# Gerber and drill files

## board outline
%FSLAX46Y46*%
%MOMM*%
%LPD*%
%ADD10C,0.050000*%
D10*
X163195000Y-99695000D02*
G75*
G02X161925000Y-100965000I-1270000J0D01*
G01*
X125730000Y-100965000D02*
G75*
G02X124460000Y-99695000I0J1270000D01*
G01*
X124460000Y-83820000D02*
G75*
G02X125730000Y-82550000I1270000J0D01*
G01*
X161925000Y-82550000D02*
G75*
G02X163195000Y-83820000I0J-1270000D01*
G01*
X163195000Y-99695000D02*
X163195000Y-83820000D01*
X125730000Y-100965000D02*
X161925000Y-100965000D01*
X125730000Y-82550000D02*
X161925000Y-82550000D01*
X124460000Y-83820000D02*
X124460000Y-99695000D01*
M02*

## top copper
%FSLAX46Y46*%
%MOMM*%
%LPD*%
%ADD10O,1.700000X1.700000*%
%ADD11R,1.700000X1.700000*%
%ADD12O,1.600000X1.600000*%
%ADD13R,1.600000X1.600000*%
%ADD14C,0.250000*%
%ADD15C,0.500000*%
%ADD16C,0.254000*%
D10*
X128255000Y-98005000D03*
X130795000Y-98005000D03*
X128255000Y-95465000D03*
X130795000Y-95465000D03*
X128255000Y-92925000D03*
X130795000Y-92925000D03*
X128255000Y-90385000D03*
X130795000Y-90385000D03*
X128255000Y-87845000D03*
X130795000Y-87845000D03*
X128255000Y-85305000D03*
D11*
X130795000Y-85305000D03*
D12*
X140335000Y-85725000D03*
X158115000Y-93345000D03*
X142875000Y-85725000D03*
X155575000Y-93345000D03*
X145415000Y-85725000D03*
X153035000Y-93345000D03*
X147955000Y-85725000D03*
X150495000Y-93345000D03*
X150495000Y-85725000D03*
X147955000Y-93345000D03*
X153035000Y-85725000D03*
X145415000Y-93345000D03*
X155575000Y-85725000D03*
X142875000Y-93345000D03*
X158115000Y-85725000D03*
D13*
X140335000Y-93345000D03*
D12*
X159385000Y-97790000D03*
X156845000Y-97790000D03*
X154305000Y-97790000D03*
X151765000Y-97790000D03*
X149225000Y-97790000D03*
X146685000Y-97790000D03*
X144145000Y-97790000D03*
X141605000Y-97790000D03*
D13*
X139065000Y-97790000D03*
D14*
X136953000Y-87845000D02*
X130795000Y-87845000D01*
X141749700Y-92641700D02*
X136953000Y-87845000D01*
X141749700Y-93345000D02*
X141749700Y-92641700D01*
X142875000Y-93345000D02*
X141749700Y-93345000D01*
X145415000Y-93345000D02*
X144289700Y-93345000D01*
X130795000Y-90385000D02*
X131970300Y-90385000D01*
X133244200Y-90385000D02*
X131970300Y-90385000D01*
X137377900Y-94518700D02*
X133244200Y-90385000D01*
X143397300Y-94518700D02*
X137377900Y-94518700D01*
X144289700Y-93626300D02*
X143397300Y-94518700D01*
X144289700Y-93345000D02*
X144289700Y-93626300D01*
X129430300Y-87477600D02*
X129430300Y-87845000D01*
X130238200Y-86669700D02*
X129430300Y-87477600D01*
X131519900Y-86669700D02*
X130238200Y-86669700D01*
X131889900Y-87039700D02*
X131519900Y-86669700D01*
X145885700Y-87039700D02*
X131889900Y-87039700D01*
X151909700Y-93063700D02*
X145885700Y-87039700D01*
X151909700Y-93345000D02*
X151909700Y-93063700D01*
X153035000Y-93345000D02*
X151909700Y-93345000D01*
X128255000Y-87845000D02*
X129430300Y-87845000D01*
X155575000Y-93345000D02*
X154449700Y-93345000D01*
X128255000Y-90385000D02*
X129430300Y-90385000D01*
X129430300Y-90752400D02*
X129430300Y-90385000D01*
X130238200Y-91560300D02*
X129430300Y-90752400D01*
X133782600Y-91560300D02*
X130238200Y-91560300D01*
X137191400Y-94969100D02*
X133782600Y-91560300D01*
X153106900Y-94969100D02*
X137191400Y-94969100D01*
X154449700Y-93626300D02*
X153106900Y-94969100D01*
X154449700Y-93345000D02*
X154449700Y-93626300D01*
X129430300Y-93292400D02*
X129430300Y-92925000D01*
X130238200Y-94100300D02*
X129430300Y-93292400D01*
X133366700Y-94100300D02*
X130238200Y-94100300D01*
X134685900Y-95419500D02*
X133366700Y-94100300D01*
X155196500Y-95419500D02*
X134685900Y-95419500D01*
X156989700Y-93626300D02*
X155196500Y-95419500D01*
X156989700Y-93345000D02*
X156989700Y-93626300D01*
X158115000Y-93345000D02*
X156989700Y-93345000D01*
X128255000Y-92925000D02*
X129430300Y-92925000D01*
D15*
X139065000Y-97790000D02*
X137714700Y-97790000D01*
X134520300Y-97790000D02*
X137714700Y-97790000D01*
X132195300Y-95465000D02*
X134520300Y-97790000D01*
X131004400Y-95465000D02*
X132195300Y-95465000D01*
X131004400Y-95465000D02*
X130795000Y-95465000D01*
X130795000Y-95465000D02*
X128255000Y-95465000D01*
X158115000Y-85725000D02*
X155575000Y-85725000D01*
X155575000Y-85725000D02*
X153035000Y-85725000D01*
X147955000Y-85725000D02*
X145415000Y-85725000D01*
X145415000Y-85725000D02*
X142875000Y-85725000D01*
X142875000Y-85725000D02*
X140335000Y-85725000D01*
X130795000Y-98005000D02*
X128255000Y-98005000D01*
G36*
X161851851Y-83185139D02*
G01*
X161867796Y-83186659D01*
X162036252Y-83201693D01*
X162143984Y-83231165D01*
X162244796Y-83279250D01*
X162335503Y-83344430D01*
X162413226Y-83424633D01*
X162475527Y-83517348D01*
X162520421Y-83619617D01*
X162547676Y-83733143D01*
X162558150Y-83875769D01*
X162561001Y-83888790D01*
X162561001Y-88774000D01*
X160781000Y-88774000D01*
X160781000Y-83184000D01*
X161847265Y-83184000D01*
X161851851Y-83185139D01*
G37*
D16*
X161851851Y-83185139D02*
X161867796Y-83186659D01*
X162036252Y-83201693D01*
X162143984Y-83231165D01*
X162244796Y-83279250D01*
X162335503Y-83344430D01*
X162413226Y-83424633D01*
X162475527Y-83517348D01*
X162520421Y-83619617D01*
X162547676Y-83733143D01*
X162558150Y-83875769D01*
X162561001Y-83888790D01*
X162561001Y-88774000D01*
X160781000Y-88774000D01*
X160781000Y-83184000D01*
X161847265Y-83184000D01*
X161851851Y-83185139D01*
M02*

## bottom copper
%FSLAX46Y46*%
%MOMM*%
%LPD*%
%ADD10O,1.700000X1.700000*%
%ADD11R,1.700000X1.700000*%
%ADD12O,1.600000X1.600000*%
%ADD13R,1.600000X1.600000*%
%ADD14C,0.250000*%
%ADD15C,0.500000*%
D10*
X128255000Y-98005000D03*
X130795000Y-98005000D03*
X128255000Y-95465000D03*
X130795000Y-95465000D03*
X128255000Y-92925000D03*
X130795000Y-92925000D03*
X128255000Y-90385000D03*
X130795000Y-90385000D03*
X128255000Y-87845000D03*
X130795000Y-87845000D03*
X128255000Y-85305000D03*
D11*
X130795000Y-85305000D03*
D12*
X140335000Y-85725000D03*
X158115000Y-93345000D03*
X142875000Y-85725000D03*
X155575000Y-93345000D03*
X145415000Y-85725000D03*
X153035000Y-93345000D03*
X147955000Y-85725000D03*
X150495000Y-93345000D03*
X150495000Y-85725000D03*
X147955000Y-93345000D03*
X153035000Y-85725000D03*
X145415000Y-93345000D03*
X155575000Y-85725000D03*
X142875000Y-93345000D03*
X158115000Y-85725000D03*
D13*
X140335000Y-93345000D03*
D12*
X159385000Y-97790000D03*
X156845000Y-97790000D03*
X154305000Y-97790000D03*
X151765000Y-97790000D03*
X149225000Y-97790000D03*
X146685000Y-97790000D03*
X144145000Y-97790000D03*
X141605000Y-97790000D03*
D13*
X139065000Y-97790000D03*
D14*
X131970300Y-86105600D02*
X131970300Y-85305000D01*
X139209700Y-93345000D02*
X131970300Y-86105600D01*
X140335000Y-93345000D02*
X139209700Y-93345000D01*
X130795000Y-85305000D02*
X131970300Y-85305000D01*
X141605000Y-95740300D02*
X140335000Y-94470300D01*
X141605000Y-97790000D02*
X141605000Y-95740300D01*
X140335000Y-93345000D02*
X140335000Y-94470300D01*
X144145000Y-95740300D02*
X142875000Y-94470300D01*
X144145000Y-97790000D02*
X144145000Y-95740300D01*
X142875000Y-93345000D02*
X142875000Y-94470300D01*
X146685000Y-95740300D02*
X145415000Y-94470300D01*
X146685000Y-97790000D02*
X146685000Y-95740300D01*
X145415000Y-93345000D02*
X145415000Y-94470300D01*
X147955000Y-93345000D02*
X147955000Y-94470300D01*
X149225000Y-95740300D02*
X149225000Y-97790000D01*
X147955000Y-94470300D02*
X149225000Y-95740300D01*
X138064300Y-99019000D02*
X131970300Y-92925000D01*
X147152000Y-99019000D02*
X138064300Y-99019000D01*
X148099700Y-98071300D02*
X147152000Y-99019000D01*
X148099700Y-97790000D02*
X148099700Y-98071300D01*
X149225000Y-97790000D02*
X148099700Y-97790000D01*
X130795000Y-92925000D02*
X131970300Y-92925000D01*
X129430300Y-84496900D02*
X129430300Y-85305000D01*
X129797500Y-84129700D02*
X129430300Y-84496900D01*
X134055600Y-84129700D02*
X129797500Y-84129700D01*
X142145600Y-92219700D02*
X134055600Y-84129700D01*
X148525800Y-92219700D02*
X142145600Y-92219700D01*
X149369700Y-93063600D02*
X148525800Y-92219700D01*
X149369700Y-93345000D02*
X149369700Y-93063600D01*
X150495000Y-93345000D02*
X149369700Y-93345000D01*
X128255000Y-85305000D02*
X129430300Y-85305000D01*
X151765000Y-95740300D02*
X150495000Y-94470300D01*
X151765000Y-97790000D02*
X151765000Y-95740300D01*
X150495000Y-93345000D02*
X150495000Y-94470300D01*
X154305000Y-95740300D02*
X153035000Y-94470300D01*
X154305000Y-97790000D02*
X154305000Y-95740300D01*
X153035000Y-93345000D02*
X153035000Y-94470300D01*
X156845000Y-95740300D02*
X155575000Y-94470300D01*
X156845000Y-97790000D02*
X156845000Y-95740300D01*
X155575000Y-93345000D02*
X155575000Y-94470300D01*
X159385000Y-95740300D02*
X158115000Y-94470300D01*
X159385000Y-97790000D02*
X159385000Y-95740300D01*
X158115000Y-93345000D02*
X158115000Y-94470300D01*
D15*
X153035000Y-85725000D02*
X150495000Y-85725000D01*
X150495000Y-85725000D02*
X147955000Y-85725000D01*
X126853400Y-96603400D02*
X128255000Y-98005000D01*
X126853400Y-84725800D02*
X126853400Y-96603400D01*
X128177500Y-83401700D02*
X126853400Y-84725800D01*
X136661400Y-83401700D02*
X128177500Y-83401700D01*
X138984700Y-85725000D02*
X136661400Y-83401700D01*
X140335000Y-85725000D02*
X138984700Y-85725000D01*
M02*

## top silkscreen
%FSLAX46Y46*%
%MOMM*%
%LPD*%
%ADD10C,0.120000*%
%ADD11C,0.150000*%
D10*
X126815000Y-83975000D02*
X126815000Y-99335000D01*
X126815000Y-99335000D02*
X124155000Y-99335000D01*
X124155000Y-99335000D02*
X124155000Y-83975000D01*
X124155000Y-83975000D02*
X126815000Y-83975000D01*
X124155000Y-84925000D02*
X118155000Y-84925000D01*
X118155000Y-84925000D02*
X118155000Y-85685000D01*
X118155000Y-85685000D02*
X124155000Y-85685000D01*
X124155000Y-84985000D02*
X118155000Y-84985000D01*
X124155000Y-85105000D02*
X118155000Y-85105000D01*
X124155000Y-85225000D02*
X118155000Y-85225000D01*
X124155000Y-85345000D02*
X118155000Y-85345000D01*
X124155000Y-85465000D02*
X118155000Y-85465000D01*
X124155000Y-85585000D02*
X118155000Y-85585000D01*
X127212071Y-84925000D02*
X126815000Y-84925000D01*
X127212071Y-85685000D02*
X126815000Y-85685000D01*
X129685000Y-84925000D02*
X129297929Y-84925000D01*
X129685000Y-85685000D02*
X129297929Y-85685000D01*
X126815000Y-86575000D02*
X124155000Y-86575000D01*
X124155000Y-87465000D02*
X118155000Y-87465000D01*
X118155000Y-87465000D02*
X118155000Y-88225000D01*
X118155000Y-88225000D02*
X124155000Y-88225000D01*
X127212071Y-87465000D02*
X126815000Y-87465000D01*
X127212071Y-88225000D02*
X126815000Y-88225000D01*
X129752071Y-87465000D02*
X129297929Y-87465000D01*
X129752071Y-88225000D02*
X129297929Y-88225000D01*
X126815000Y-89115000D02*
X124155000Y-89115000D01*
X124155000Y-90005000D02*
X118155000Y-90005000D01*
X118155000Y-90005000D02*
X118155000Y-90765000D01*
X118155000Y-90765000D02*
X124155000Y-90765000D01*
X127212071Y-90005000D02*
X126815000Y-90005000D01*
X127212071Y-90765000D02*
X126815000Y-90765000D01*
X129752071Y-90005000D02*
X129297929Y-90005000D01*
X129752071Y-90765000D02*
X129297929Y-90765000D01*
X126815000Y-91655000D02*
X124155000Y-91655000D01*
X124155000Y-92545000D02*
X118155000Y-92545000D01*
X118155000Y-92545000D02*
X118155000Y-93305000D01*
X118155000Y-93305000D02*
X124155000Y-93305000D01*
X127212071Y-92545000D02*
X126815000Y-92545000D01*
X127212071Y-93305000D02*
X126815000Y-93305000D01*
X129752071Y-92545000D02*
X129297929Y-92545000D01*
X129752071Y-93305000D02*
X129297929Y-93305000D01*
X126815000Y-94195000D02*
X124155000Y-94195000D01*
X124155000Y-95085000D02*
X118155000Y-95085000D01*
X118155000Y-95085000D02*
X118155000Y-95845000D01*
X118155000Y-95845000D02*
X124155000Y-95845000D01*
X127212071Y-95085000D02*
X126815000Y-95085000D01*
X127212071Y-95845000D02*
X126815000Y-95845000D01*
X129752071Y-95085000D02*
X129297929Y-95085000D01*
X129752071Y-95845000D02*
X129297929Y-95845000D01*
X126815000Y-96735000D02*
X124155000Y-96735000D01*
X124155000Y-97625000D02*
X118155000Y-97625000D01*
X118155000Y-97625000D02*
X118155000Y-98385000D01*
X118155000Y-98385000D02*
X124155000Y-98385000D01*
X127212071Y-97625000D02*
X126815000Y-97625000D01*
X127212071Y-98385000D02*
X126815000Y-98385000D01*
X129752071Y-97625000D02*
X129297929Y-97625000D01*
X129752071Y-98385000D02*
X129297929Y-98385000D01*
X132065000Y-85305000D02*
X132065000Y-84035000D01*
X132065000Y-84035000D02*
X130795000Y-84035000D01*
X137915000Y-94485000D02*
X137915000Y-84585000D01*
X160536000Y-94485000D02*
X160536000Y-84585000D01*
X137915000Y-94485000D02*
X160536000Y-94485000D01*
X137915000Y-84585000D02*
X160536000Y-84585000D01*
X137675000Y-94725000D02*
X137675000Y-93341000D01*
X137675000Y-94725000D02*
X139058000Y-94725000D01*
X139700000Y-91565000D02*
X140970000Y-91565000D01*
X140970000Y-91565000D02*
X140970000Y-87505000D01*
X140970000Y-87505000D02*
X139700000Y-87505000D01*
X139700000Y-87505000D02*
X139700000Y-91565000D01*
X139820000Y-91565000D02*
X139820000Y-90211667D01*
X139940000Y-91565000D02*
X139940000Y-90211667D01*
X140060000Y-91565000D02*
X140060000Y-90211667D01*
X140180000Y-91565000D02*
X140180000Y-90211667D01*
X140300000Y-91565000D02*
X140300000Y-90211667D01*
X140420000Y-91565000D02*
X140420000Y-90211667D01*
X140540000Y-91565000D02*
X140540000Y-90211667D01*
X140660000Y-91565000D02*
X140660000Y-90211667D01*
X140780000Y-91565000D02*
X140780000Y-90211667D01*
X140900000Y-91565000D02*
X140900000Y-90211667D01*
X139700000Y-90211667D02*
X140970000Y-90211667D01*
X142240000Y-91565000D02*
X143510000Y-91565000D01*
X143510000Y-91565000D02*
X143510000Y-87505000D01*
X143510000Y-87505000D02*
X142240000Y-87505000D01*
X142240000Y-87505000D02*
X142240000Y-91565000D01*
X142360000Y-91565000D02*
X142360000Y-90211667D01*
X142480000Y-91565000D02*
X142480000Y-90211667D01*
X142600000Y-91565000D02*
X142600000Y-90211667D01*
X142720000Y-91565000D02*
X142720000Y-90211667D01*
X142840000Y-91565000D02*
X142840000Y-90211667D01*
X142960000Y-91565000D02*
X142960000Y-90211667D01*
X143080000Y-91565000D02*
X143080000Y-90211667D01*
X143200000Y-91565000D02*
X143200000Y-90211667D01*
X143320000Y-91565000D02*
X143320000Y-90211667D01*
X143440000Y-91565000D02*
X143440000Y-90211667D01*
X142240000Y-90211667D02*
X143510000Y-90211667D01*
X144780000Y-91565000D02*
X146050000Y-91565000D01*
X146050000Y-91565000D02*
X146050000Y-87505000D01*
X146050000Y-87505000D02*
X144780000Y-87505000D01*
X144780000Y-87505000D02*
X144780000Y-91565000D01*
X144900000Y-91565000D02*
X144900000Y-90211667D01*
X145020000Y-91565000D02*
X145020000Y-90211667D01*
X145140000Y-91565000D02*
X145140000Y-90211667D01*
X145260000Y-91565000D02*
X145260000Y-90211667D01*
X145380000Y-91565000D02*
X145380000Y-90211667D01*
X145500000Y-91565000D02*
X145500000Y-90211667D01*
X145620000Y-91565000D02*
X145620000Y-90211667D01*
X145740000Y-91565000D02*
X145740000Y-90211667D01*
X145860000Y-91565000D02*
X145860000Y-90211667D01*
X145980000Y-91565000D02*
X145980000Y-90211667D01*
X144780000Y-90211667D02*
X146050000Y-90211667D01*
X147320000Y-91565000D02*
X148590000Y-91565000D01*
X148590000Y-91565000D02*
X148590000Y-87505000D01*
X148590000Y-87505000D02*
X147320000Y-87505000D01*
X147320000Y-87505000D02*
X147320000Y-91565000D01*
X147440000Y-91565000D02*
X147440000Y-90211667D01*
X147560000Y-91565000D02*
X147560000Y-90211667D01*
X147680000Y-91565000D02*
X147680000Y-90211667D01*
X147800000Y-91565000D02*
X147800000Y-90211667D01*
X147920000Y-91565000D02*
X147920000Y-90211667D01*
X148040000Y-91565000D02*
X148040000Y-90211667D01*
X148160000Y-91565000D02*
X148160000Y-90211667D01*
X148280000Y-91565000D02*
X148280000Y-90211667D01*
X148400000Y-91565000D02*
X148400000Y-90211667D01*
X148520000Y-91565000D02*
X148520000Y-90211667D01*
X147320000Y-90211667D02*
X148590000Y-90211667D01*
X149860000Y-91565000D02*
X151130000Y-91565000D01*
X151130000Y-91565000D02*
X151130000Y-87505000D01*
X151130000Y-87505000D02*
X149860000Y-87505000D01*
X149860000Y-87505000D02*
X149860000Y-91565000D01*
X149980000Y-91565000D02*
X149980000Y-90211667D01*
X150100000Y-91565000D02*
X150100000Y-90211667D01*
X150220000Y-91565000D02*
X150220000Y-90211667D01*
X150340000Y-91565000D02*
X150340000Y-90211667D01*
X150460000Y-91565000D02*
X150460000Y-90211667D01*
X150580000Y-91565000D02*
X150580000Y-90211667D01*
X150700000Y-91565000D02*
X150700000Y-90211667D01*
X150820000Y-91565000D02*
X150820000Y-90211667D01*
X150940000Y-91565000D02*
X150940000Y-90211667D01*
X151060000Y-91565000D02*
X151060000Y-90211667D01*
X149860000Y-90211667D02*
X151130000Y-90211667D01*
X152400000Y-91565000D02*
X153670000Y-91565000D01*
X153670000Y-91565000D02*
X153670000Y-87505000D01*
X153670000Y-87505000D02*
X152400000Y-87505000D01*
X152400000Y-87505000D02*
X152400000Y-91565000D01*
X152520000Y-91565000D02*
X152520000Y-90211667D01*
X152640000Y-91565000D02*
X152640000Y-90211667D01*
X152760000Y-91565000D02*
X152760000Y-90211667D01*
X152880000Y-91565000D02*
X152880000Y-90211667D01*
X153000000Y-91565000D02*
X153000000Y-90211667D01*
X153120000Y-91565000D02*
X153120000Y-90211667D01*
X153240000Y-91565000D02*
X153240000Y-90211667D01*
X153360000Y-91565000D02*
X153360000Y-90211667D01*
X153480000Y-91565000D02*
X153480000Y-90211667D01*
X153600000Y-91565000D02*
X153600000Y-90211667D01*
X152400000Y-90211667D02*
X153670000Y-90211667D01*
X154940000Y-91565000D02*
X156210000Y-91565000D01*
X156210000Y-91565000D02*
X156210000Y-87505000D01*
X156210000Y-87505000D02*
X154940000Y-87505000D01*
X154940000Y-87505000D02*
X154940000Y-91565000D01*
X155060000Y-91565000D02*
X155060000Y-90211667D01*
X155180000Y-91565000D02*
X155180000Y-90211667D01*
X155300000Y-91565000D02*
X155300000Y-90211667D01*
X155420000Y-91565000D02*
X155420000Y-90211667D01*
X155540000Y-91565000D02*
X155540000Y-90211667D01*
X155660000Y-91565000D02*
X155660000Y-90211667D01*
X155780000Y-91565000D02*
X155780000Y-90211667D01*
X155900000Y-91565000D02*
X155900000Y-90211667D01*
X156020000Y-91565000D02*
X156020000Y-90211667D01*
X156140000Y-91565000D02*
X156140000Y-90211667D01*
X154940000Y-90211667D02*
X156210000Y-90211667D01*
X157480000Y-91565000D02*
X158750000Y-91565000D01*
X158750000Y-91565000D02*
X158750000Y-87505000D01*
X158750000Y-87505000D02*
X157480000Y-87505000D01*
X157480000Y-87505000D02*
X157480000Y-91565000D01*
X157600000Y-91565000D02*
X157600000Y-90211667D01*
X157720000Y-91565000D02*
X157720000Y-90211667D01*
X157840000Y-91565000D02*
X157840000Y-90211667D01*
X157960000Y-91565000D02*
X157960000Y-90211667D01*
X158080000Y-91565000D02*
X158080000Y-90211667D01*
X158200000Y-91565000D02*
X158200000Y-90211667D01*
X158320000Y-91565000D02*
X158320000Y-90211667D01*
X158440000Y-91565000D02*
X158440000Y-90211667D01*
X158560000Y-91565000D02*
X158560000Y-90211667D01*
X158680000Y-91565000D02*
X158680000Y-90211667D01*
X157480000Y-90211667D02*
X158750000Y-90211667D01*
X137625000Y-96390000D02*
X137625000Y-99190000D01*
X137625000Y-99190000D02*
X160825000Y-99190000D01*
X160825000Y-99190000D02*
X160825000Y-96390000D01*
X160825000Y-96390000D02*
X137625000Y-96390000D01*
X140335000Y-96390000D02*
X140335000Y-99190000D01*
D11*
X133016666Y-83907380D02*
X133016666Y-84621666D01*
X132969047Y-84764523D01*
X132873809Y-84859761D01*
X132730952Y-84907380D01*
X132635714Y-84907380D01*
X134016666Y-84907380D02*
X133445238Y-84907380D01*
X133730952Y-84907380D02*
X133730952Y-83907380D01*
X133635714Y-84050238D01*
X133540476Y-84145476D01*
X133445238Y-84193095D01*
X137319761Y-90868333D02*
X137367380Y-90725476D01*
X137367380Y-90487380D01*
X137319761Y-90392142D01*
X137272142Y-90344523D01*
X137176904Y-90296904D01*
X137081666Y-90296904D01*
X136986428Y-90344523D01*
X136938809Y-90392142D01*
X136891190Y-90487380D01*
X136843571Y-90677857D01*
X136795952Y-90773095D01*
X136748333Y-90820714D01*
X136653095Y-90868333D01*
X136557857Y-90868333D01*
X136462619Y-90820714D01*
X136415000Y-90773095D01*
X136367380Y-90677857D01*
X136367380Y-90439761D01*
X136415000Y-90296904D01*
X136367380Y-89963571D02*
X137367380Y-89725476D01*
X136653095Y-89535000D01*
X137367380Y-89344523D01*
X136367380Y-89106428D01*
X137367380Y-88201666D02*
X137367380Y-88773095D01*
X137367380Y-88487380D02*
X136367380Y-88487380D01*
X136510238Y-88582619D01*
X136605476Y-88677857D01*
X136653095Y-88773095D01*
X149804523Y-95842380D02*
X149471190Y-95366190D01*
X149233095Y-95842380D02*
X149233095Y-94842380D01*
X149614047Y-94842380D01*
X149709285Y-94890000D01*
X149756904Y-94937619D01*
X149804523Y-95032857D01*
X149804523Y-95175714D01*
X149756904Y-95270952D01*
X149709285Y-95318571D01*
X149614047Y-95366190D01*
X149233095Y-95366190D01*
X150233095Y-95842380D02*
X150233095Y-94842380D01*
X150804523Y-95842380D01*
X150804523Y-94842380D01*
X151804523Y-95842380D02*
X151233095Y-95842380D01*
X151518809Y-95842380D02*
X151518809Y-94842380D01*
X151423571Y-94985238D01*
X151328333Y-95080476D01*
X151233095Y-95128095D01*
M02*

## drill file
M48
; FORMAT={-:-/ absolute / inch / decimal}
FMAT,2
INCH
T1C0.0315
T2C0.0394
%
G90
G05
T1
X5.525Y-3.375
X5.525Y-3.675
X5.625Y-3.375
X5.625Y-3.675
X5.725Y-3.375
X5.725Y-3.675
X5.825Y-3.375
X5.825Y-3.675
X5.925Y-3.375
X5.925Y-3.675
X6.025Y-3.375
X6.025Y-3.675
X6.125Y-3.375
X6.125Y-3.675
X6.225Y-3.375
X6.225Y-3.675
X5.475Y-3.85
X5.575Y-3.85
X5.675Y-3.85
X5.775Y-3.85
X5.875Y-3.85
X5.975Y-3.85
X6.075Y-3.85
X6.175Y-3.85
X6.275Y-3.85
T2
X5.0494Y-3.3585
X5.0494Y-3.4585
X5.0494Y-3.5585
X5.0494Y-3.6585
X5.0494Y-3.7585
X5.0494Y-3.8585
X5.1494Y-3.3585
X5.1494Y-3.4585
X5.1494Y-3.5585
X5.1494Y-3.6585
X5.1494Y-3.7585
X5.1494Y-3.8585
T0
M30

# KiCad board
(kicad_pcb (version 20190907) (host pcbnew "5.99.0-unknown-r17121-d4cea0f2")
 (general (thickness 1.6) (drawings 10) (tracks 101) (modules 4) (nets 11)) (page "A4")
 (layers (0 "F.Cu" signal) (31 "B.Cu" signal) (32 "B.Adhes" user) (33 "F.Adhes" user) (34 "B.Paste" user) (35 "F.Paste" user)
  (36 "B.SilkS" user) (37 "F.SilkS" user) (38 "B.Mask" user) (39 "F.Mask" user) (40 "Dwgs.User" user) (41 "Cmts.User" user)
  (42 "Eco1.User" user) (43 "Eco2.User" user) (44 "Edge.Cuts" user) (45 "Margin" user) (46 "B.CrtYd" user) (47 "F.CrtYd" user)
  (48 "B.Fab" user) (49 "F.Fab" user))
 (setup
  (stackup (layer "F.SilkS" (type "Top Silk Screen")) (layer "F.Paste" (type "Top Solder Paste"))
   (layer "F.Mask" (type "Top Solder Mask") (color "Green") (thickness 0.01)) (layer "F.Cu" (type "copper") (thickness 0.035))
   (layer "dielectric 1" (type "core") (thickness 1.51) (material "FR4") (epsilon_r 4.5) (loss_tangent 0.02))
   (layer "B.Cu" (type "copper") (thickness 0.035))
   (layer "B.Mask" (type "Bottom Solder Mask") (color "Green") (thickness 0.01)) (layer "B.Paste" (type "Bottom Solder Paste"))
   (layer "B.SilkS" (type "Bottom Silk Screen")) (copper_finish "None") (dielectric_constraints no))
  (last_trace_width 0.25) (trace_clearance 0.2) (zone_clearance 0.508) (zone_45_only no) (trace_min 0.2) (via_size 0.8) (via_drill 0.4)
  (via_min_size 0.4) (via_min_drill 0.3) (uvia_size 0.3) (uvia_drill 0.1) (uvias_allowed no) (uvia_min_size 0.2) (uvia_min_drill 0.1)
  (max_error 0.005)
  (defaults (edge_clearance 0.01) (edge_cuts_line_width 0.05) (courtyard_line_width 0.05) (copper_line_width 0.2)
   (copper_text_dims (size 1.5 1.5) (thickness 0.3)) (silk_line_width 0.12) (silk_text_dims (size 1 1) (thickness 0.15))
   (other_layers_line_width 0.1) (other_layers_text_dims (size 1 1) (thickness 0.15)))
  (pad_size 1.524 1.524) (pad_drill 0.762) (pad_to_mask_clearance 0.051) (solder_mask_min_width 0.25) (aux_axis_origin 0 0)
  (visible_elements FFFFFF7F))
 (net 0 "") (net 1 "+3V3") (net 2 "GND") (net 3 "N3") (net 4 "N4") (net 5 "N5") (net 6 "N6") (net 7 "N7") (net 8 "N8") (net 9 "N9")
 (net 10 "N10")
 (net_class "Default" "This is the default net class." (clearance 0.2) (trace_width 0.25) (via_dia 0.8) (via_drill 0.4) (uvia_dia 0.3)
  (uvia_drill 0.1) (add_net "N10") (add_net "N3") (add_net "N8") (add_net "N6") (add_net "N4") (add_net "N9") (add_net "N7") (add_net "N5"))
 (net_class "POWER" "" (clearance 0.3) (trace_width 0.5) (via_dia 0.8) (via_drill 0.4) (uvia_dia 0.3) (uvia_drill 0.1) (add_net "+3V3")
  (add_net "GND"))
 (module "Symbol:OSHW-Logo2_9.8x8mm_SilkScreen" (layer "B.Cu") (at 135.255 91.694 -90)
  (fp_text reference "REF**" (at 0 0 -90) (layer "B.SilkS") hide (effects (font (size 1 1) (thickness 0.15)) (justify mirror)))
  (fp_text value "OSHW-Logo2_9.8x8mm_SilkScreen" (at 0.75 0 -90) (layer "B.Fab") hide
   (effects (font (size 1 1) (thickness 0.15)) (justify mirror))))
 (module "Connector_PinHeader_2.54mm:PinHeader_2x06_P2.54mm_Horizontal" (layer "F.Cu") (at 125.095 90.805)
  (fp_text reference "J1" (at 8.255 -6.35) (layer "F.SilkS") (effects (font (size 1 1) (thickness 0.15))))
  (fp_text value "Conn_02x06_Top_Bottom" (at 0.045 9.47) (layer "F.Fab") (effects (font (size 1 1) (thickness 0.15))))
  (fp_line (start 1.72 -6.83) (end 1.72 8.53) (layer "F.SilkS") (width 0.12))
  (fp_line (start 1.72 8.53) (end -0.94 8.53) (layer "F.SilkS") (width 0.12))
  (fp_line (start -0.94 8.53) (end -0.94 -6.83) (layer "F.SilkS") (width 0.12))
  (fp_line (start -0.94 -6.83) (end 1.72 -6.83) (layer "F.SilkS") (width 0.12))
  (fp_line (start -0.94 -5.88) (end -6.94 -5.88) (layer "F.SilkS") (width 0.12))
  (fp_line (start -6.94 -5.88) (end -6.94 -5.12) (layer "F.SilkS") (width 0.12))
  (fp_line (start -6.94 -5.12) (end -0.94 -5.12) (layer "F.SilkS") (width 0.12))
  (fp_line (start -0.94 -5.82) (end -6.94 -5.82) (layer "F.SilkS") (width 0.12))
  (fp_line (start -0.94 -5.7) (end -6.94 -5.7) (layer "F.SilkS") (width 0.12))
  (fp_line (start -0.94 -5.58) (end -6.94 -5.58) (layer "F.SilkS") (width 0.12))
  (fp_line (start -0.94 -5.46) (end -6.94 -5.46) (layer "F.SilkS") (width 0.12))
  (fp_line (start -0.94 -5.34) (end -6.94 -5.34) (layer "F.SilkS") (width 0.12))
  (fp_line (start -0.94 -5.22) (end -6.94 -5.22) (layer "F.SilkS") (width 0.12))
  (fp_line (start 2.117071 -5.88) (end 1.72 -5.88) (layer "F.SilkS") (width 0.12))
  (fp_line (start 2.117071 -5.12) (end 1.72 -5.12) (layer "F.SilkS") (width 0.12))
  (fp_line (start 4.59 -5.88) (end 4.202929 -5.88) (layer "F.SilkS") (width 0.12))
  (fp_line (start 4.59 -5.12) (end 4.202929 -5.12) (layer "F.SilkS") (width 0.12))
  (fp_line (start 1.72 -4.23) (end -0.94 -4.23) (layer "F.SilkS") (width 0.12))
  (fp_line (start -0.94 -3.34) (end -6.94 -3.34) (layer "F.SilkS") (width 0.12))
  (fp_line (start -6.94 -3.34) (end -6.94 -2.58) (layer "F.SilkS") (width 0.12))
  (fp_line (start -6.94 -2.58) (end -0.94 -2.58) (layer "F.SilkS") (width 0.12))
  (fp_line (start 2.117071 -3.34) (end 1.72 -3.34) (layer "F.SilkS") (width 0.12))
  (fp_line (start 2.117071 -2.58) (end 1.72 -2.58) (layer "F.SilkS") (width 0.12))
  (fp_line (start 4.657071 -3.34) (end 4.202929 -3.34) (layer "F.SilkS") (width 0.12))
  (fp_line (start 4.657071 -2.58) (end 4.202929 -2.58) (layer "F.SilkS") (width 0.12))
  (fp_line (start 1.72 -1.69) (end -0.94 -1.69) (layer "F.SilkS") (width 0.12))
  (fp_line (start -0.94 -0.8) (end -6.94 -0.8) (layer "F.SilkS") (width 0.12))
  (fp_line (start -6.94 -0.8) (end -6.94 -0.04) (layer "F.SilkS") (width 0.12))
  (fp_line (start -6.94 -0.04) (end -0.94 -0.04) (layer "F.SilkS") (width 0.12))
  (fp_line (start 2.117071 -0.8) (end 1.72 -0.8) (layer "F.SilkS") (width 0.12))
  (fp_line (start 2.117071 -0.04) (end 1.72 -0.04) (layer "F.SilkS") (width 0.12))
  (fp_line (start 4.657071 -0.8) (end 4.202929 -0.8) (layer "F.SilkS") (width 0.12))
  (fp_line (start 4.657071 -0.04) (end 4.202929 -0.04) (layer "F.SilkS") (width 0.12))
  (fp_line (start 1.72 0.85) (end -0.94 0.85) (layer "F.SilkS") (width 0.12))
  (fp_line (start -0.94 1.74) (end -6.94 1.74) (layer "F.SilkS") (width 0.12))
  (fp_line (start -6.94 1.74) (end -6.94 2.5) (layer "F.SilkS") (width 0.12))
  (fp_line (start -6.94 2.5) (end -0.94 2.5) (layer "F.SilkS") (width 0.12))
  (fp_line (start 2.117071 1.74) (end 1.72 1.74) (layer "F.SilkS") (width 0.12))
  (fp_line (start 2.117071 2.5) (end 1.72 2.5) (layer "F.SilkS") (width 0.12))
  (fp_line (start 4.657071 1.74) (end 4.202929 1.74) (layer "F.SilkS") (width 0.12))
  (fp_line (start 4.657071 2.5) (end 4.202929 2.5) (layer "F.SilkS") (width 0.12))
  (fp_line (start 1.72 3.39) (end -0.94 3.39) (layer "F.SilkS") (width 0.12))
  (fp_line (start -0.94 4.28) (end -6.94 4.28) (layer "F.SilkS") (width 0.12))
  (fp_line (start -6.94 4.28) (end -6.94 5.04) (layer "F.SilkS") (width 0.12))
  (fp_line (start -6.94 5.04) (end -0.94 5.04) (layer "F.SilkS") (width 0.12))
  (fp_line (start 2.117071 4.28) (end 1.72 4.28) (layer "F.SilkS") (width 0.12))
  (fp_line (start 2.117071 5.04) (end 1.72 5.04) (layer "F.SilkS") (width 0.12))
  (fp_line (start 4.657071 4.28) (end 4.202929 4.28) (layer "F.SilkS") (width 0.12))
  (fp_line (start 4.657071 5.04) (end 4.202929 5.04) (layer "F.SilkS") (width 0.12))
  (fp_line (start 1.72 5.93) (end -0.94 5.93) (layer "F.SilkS") (width 0.12))
  (fp_line (start -0.94 6.82) (end -6.94 6.82) (layer "F.SilkS") (width 0.12))
  (fp_line (start -6.94 6.82) (end -6.94 7.58) (layer "F.SilkS") (width 0.12))
  (fp_line (start -6.94 7.58) (end -0.94 7.58) (layer "F.SilkS") (width 0.12))
  (fp_line (start 2.117071 6.82) (end 1.72 6.82) (layer "F.SilkS") (width 0.12))
  (fp_line (start 2.117071 7.58) (end 1.72 7.58) (layer "F.SilkS") (width 0.12))
  (fp_line (start 4.657071 6.82) (end 4.202929 6.82) (layer "F.SilkS") (width 0.12))
  (fp_line (start 4.657071 7.58) (end 4.202929 7.58) (layer "F.SilkS") (width 0.12))
  (fp_line (start 6.97 -5.5) (end 6.97 -6.77) (layer "F.SilkS") (width 0.12))
  (fp_line (start 6.97 -6.77) (end 5.7 -6.77) (layer "F.SilkS") (width 0.12))
  (pad "12" thru_hole oval (at 3.16 7.2) (size 1.7 1.7) (drill 1) (layers *.Cu *.Mask) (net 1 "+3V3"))
  (pad "6" thru_hole oval (at 5.7 7.2) (size 1.7 1.7) (drill 1) (layers *.Cu *.Mask) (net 1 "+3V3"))
  (pad "11" thru_hole oval (at 3.16 4.66) (size 1.7 1.7) (drill 1) (layers *.Cu *.Mask) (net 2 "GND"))
  (pad "5" thru_hole oval (at 5.7 4.66) (size 1.7 1.7) (drill 1) (layers *.Cu *.Mask) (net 2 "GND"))
  (pad "10" thru_hole oval (at 3.16 2.12) (size 1.7 1.7) (drill 1) (layers *.Cu *.Mask) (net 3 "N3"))
  (pad "4" thru_hole oval (at 5.7 2.12) (size 1.7 1.7) (drill 1) (layers *.Cu *.Mask) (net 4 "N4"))
  (pad "9" thru_hole oval (at 3.16 -0.42) (size 1.7 1.7) (drill 1) (layers *.Cu *.Mask) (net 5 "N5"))
  (pad "3" thru_hole oval (at 5.7 -0.42) (size 1.7 1.7) (drill 1) (layers *.Cu *.Mask) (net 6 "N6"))
  (pad "8" thru_hole oval (at 3.16 -2.96) (size 1.7 1.7) (drill 1) (layers *.Cu *.Mask) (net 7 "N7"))
  (pad "2" thru_hole oval (at 5.7 -2.96) (size 1.7 1.7) (drill 1) (layers *.Cu *.Mask) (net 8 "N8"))
  (pad "7" thru_hole oval (at 3.16 -5.5) (size 1.7 1.7) (drill 1) (layers *.Cu *.Mask) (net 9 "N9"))
  (pad "1" thru_hole rect (at 5.7 -5.5) (size 1.7 1.7) (drill 1) (layers *.Cu *.Mask) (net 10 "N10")))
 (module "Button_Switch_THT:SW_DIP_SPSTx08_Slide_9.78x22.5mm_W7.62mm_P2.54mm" (layer "F.Cu") (at 140.335 93.345 90)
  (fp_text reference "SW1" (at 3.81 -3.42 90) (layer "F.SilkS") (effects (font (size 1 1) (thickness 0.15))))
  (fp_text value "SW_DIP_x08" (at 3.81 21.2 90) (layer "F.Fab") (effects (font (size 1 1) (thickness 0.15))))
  (fp_line (start -1.14 -2.42) (end 8.76 -2.42) (layer "F.SilkS") (width 0.12))
  (fp_line (start -1.14 20.201) (end 8.76 20.201) (layer "F.SilkS") (width 0.12))
  (fp_line (start -1.14 -2.42) (end -1.14 20.201) (layer "F.SilkS") (width 0.12))
  (fp_line (start 8.76 -2.42) (end 8.76 20.201) (layer "F.SilkS") (width 0.12))
  (fp_line (start -1.38 -2.66) (end 0.004 -2.66) (layer "F.SilkS") (width 0.12))
  (fp_line (start -1.38 -2.66) (end -1.38 -1.277) (layer "F.SilkS") (width 0.12))
  (fp_line (start 1.78 -0.635) (end 1.78 0.635) (layer "F.SilkS") (width 0.12))
  (fp_line (start 1.78 0.635) (end 5.84 0.635) (layer "F.SilkS") (width 0.12))
  (fp_line (start 5.84 0.635) (end 5.84 -0.635) (layer "F.SilkS") (width 0.12))
  (fp_line (start 5.84 -0.635) (end 1.78 -0.635) (layer "F.SilkS") (width 0.12))
  (fp_line (start 1.78 -0.515) (end 3.133333 -0.515) (layer "F.SilkS") (width 0.12))
  (fp_line (start 1.78 -0.395) (end 3.133333 -0.395) (layer "F.SilkS") (width 0.12))
  (fp_line (start 1.78 -0.275) (end 3.133333 -0.275) (layer "F.SilkS") (width 0.12))
  (fp_line (start 1.78 -0.155) (end 3.133333 -0.155) (layer "F.SilkS") (width 0.12))
  (fp_line (start 1.78 -0.035) (end 3.133333 -0.035) (layer "F.SilkS") (width 0.12))
  (fp_line (start 1.78 0.085) (end 3.133333 0.085) (layer "F.SilkS") (width 0.12))
  (fp_line (start 1.78 0.205) (end 3.133333 0.205) (layer "F.SilkS") (width 0.12))
  (fp_line (start 1.78 0.325) (end 3.133333 0.325) (layer "F.SilkS") (width 0.12))
  (fp_line (start 1.78 0.445) (end 3.133333 0.445) (layer "F.SilkS") (width 0.12))
  (fp_line (start 1.78 0.565) (end 3.133333 0.565) (layer "F.SilkS") (width 0.12))
  (fp_line (start 3.133333 -0.635) (end 3.133333 0.635) (layer "F.SilkS") (width 0.12))
  (fp_line (start 1.78 1.905) (end 1.78 3.175) (layer "F.SilkS") (width 0.12))
  (fp_line (start 1.78 3.175) (end 5.84 3.175) (layer "F.SilkS") (width 0.12))
  (fp_line (start 5.84 3.175) (end 5.84 1.905) (layer "F.SilkS") (width 0.12))
  (fp_line (start 5.84 1.905) (end 1.78 1.905) (layer "F.SilkS") (width 0.12))
  (fp_line (start 1.78 2.025) (end 3.133333 2.025) (layer "F.SilkS") (width 0.12))
  (fp_line (start 1.78 2.145) (end 3.133333 2.145) (layer "F.SilkS") (width 0.12))
  (fp_line (start 1.78 2.265) (end 3.133333 2.265) (layer "F.SilkS") (width 0.12))
  (fp_line (start 1.78 2.385) (end 3.133333 2.385) (layer "F.SilkS") (width 0.12))
  (fp_line (start 1.78 2.505) (end 3.133333 2.505) (layer "F.SilkS") (width 0.12))
  (fp_line (start 1.78 2.625) (end 3.133333 2.625) (layer "F.SilkS") (width 0.12))
  (fp_line (start 1.78 2.745) (end 3.133333 2.745) (layer "F.SilkS") (width 0.12))
  (fp_line (start 1.78 2.865) (end 3.133333 2.865) (layer "F.SilkS") (width 0.12))
  (fp_line (start 1.78 2.985) (end 3.133333 2.985) (layer "F.SilkS") (width 0.12))
  (fp_line (start 1.78 3.105) (end 3.133333 3.105) (layer "F.SilkS") (width 0.12))
  (fp_line (start 3.133333 1.905) (end 3.133333 3.175) (layer "F.SilkS") (width 0.12))
  (fp_line (start 1.78 4.445) (end 1.78 5.715) (layer "F.SilkS") (width 0.12))
  (fp_line (start 1.78 5.715) (end 5.84 5.715) (layer "F.SilkS") (width 0.12))
  (fp_line (start 5.84 5.715) (end 5.84 4.445) (layer "F.SilkS") (width 0.12))
  (fp_line (start 5.84 4.445) (end 1.78 4.445) (layer "F.SilkS") (width 0.12))
  (fp_line (start 1.78 4.565) (end 3.133333 4.565) (layer "F.SilkS") (width 0.12))
  (fp_line (start 1.78 4.685) (end 3.133333 4.685) (layer "F.SilkS") (width 0.12))
  (fp_line (start 1.78 4.805) (end 3.133333 4.805) (layer "F.SilkS") (width 0.12))
  (fp_line (start 1.78 4.925) (end 3.133333 4.925) (layer "F.SilkS") (width 0.12))
  (fp_line (start 1.78 5.045) (end 3.133333 5.045) (layer "F.SilkS") (width 0.12))
  (fp_line (start 1.78 5.165) (end 3.133333 5.165) (layer "F.SilkS") (width 0.12))
  (fp_line (start 1.78 5.285) (end 3.133333 5.285) (layer "F.SilkS") (width 0.12))
  (fp_line (start 1.78 5.405) (end 3.133333 5.405) (layer "F.SilkS") (width 0.12))
  (fp_line (start 1.78 5.525) (end 3.133333 5.525) (layer "F.SilkS") (width 0.12))
  (fp_line (start 1.78 5.645) (end 3.133333 5.645) (layer "F.SilkS") (width 0.12))
  (fp_line (start 3.133333 4.445) (end 3.133333 5.715) (layer "F.SilkS") (width 0.12))
  (fp_line (start 1.78 6.985) (end 1.78 8.255) (layer "F.SilkS") (width 0.12))
  (fp_line (start 1.78 8.255) (end 5.84 8.255) (layer "F.SilkS") (width 0.12))
  (fp_line (start 5.84 8.255) (end 5.84 6.985) (layer "F.SilkS") (width 0.12))
  (fp_line (start 5.84 6.985) (end 1.78 6.985) (layer "F.SilkS") (width 0.12))
  (fp_line (start 1.78 7.105) (end 3.133333 7.105) (layer "F.SilkS") (width 0.12))
  (fp_line (start 1.78 7.225) (end 3.133333 7.225) (layer "F.SilkS") (width 0.12))
  (fp_line (start 1.78 7.345) (end 3.133333 7.345) (layer "F.SilkS") (width 0.12))
  (fp_line (start 1.78 7.465) (end 3.133333 7.465) (layer "F.SilkS") (width 0.12))
  (fp_line (start 1.78 7.585) (end 3.133333 7.585) (layer "F.SilkS") (width 0.12))
  (fp_line (start 1.78 7.705) (end 3.133333 7.705) (layer "F.SilkS") (width 0.12))
  (fp_line (start 1.78 7.825) (end 3.133333 7.825) (layer "F.SilkS") (width 0.12))
  (fp_line (start 1.78 7.945) (end 3.133333 7.945) (layer "F.SilkS") (width 0.12))
  (fp_line (start 1.78 8.065) (end 3.133333 8.065) (layer "F.SilkS") (width 0.12))
  (fp_line (start 1.78 8.185) (end 3.133333 8.185) (layer "F.SilkS") (width 0.12))
  (fp_line (start 3.133333 6.985) (end 3.133333 8.255) (layer "F.SilkS") (width 0.12))
  (fp_line (start 1.78 9.525) (end 1.78 10.795) (layer "F.SilkS") (width 0.12))
  (fp_line (start 1.78 10.795) (end 5.84 10.795) (layer "F.SilkS") (width 0.12))
  (fp_line (start 5.84 10.795) (end 5.84 9.525) (layer "F.SilkS") (width 0.12))
  (fp_line (start 5.84 9.525) (end 1.78 9.525) (layer "F.SilkS") (width 0.12))
  (fp_line (start 1.78 9.645) (end 3.133333 9.645) (layer "F.SilkS") (width 0.12))
  (fp_line (start 1.78 9.765) (end 3.133333 9.765) (layer "F.SilkS") (width 0.12))
  (fp_line (start 1.78 9.885) (end 3.133333 9.885) (layer "F.SilkS") (width 0.12))
  (fp_line (start 1.78 10.005) (end 3.133333 10.005) (layer "F.SilkS") (width 0.12))
  (fp_line (start 1.78 10.125) (end 3.133333 10.125) (layer "F.SilkS") (width 0.12))
  (fp_line (start 1.78 10.245) (end 3.133333 10.245) (layer "F.SilkS") (width 0.12))
  (fp_line (start 1.78 10.365) (end 3.133333 10.365) (layer "F.SilkS") (width 0.12))
  (fp_line (start 1.78 10.485) (end 3.133333 10.485) (layer "F.SilkS") (width 0.12))
  (fp_line (start 1.78 10.605) (end 3.133333 10.605) (layer "F.SilkS") (width 0.12))
  (fp_line (start 1.78 10.725) (end 3.133333 10.725) (layer "F.SilkS") (width 0.12))
  (fp_line (start 3.133333 9.525) (end 3.133333 10.795) (layer "F.SilkS") (width 0.12))
  (fp_line (start 1.78 12.065) (end 1.78 13.335) (layer "F.SilkS") (width 0.12))
  (fp_line (start 1.78 13.335) (end 5.84 13.335) (layer "F.SilkS") (width 0.12))
  (fp_line (start 5.84 13.335) (end 5.84 12.065) (layer "F.SilkS") (width 0.12))
  (fp_line (start 5.84 12.065) (end 1.78 12.065) (layer "F.SilkS") (width 0.12))
  (fp_line (start 1.78 12.185) (end 3.133333 12.185) (layer "F.SilkS") (width 0.12))
  (fp_line (start 1.78 12.305) (end 3.133333 12.305) (layer "F.SilkS") (width 0.12))
  (fp_line (start 1.78 12.425) (end 3.133333 12.425) (layer "F.SilkS") (width 0.12))
  (fp_line (start 1.78 12.545) (end 3.133333 12.545) (layer "F.SilkS") (width 0.12))
  (fp_line (start 1.78 12.665) (end 3.133333 12.665) (layer "F.SilkS") (width 0.12))
  (fp_line (start 1.78 12.785) (end 3.133333 12.785) (layer "F.SilkS") (width 0.12))
  (fp_line (start 1.78 12.905) (end 3.133333 12.905) (layer "F.SilkS") (width 0.12))
  (fp_line (start 1.78 13.025) (end 3.133333 13.025) (layer "F.SilkS") (width 0.12))
  (fp_line (start 1.78 13.145) (end 3.133333 13.145) (layer "F.SilkS") (width 0.12))
  (fp_line (start 1.78 13.265) (end 3.133333 13.265) (layer "F.SilkS") (width 0.12))
  (fp_line (start 3.133333 12.065) (end 3.133333 13.335) (layer "F.SilkS") (width 0.12))
  (fp_line (start 1.78 14.605) (end 1.78 15.875) (layer "F.SilkS") (width 0.12))
  (fp_line (start 1.78 15.875) (end 5.84 15.875) (layer "F.SilkS") (width 0.12))
  (fp_line (start 5.84 15.875) (end 5.84 14.605) (layer "F.SilkS") (width 0.12))
  (fp_line (start 5.84 14.605) (end 1.78 14.605) (layer "F.SilkS") (width 0.12))
  (fp_line (start 1.78 14.725) (end 3.133333 14.725) (layer "F.SilkS") (width 0.12))
  (fp_line (start 1.78 14.845) (end 3.133333 14.845) (layer "F.SilkS") (width 0.12))
  (fp_line (start 1.78 14.965) (end 3.133333 14.965) (layer "F.SilkS") (width 0.12))
  (fp_line (start 1.78 15.085) (end 3.133333 15.085) (layer "F.SilkS") (width 0.12))
  (fp_line (start 1.78 15.205) (end 3.133333 15.205) (layer "F.SilkS") (width 0.12))
  (fp_line (start 1.78 15.325) (end 3.133333 15.325) (layer "F.SilkS") (width 0.12))
  (fp_line (start 1.78 15.445) (end 3.133333 15.445) (layer "F.SilkS") (width 0.12))
  (fp_line (start 1.78 15.565) (end 3.133333 15.565) (layer "F.SilkS") (width 0.12))
  (fp_line (start 1.78 15.685) (end 3.133333 15.685) (layer "F.SilkS") (width 0.12))
  (fp_line (start 1.78 15.805) (end 3.133333 15.805) (layer "F.SilkS") (width 0.12))
  (fp_line (start 3.133333 14.605) (end 3.133333 15.875) (layer "F.SilkS") (width 0.12))
  (fp_line (start 1.78 17.145) (end 1.78 18.415) (layer "F.SilkS") (width 0.12))
  (fp_line (start 1.78 18.415) (end 5.84 18.415) (layer "F.SilkS") (width 0.12))
  (fp_line (start 5.84 18.415) (end 5.84 17.145) (layer "F.SilkS") (width 0.12))
  (fp_line (start 5.84 17.145) (end 1.78 17.145) (layer "F.SilkS") (width 0.12))
  (fp_line (start 1.78 17.265) (end 3.133333 17.265) (layer "F.SilkS") (width 0.12))
  (fp_line (start 1.78 17.385) (end 3.133333 17.385) (layer "F.SilkS") (width 0.12))
  (fp_line (start 1.78 17.505) (end 3.133333 17.505) (layer "F.SilkS") (width 0.12))
  (fp_line (start 1.78 17.625) (end 3.133333 17.625) (layer "F.SilkS") (width 0.12))
  (fp_line (start 1.78 17.745) (end 3.133333 17.745) (layer "F.SilkS") (width 0.12))
  (fp_line (start 1.78 17.865) (end 3.133333 17.865) (layer "F.SilkS") (width 0.12))
  (fp_line (start 1.78 17.985) (end 3.133333 17.985) (layer "F.SilkS") (width 0.12))
  (fp_line (start 1.78 18.105) (end 3.133333 18.105) (layer "F.SilkS") (width 0.12))
  (fp_line (start 1.78 18.225) (end 3.133333 18.225) (layer "F.SilkS") (width 0.12))
  (fp_line (start 1.78 18.345) (end 3.133333 18.345) (layer "F.SilkS") (width 0.12))
  (fp_line (start 3.133333 17.145) (end 3.133333 18.415) (layer "F.SilkS") (width 0.12))
  (pad "16" thru_hole oval (at 7.62 0 90) (size 1.6 1.6) (drill 0.8) (layers *.Cu *.Mask) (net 1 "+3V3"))
  (pad "8" thru_hole oval (at 0 17.78 90) (size 1.6 1.6) (drill 0.8) (layers *.Cu *.Mask) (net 3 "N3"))
  (pad "15" thru_hole oval (at 7.62 2.54 90) (size 1.6 1.6) (drill 0.8) (layers *.Cu *.Mask) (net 1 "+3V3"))
  (pad "7" thru_hole oval (at 0 15.24 90) (size 1.6 1.6) (drill 0.8) (layers *.Cu *.Mask) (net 5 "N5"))
  (pad "14" thru_hole oval (at 7.62 5.08 90) (size 1.6 1.6) (drill 0.8) (layers *.Cu *.Mask) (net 1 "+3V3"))
  (pad "6" thru_hole oval (at 0 12.7 90) (size 1.6 1.6) (drill 0.8) (layers *.Cu *.Mask) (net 7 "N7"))
  (pad "13" thru_hole oval (at 7.62 7.62 90) (size 1.6 1.6) (drill 0.8) (layers *.Cu *.Mask) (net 1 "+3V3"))
  (pad "5" thru_hole oval (at 0 10.16 90) (size 1.6 1.6) (drill 0.8) (layers *.Cu *.Mask) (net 9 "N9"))
  (pad "12" thru_hole oval (at 7.62 10.16 90) (size 1.6 1.6) (drill 0.8) (layers *.Cu *.Mask) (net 1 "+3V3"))
  (pad "4" thru_hole oval (at 0 7.62 90) (size 1.6 1.6) (drill 0.8) (layers *.Cu *.Mask) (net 4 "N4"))
  (pad "11" thru_hole oval (at 7.62 12.7 90) (size 1.6 1.6) (drill 0.8) (layers *.Cu *.Mask) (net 1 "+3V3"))
  (pad "3" thru_hole oval (at 0 5.08 90) (size 1.6 1.6) (drill 0.8) (layers *.Cu *.Mask) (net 6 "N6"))
  (pad "10" thru_hole oval (at 7.62 15.24 90) (size 1.6 1.6) (drill 0.8) (layers *.Cu *.Mask) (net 1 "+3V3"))
  (pad "2" thru_hole oval (at 0 2.54 90) (size 1.6 1.6) (drill 0.8) (layers *.Cu *.Mask) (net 8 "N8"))
  (pad "9" thru_hole oval (at 7.62 17.78 90) (size 1.6 1.6) (drill 0.8) (layers *.Cu *.Mask) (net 1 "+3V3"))
  (pad "1" thru_hole rect (at 0 0 90) (size 1.6 1.6) (drill 0.8) (layers *.Cu *.Mask) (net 10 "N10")))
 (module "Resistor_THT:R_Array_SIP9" (layer "F.Cu") (at 139.065 97.79)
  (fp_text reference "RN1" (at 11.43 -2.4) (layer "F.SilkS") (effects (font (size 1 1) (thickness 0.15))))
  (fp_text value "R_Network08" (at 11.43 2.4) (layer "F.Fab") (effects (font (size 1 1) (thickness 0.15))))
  (fp_line (start -1.44 -1.4) (end -1.44 1.4) (layer "F.SilkS") (width 0.12))
  (fp_line (start -1.44 1.4) (end 21.76 1.4) (layer "F.SilkS") (width 0.12))
  (fp_line (start 21.76 1.4) (end 21.76 -1.4) (layer "F.SilkS") (width 0.12))
  (fp_line (start 21.76 -1.4) (end -1.44 -1.4) (layer "F.SilkS") (width 0.12))
  (fp_line (start 1.27 -1.4) (end 1.27 1.4) (layer "F.SilkS") (width 0.12))
  (pad "9" thru_hole oval (at 20.32 0) (size 1.6 1.6) (drill 0.8) (layers *.Cu *.Mask) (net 3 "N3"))
  (pad "8" thru_hole oval (at 17.78 0) (size 1.6 1.6) (drill 0.8) (layers *.Cu *.Mask) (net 5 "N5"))
  (pad "7" thru_hole oval (at 15.24 0) (size 1.6 1.6) (drill 0.8) (layers *.Cu *.Mask) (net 7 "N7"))
  (pad "6" thru_hole oval (at 12.7 0) (size 1.6 1.6) (drill 0.8) (layers *.Cu *.Mask) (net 9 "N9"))
  (pad "5" thru_hole oval (at 10.16 0) (size 1.6 1.6) (drill 0.8) (layers *.Cu *.Mask) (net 4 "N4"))
  (pad "4" thru_hole oval (at 7.62 0) (size 1.6 1.6) (drill 0.8) (layers *.Cu *.Mask) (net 6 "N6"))
  (pad "3" thru_hole oval (at 5.08 0) (size 1.6 1.6) (drill 0.8) (layers *.Cu *.Mask) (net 8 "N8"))
  (pad "2" thru_hole oval (at 2.54 0) (size 1.6 1.6) (drill 0.8) (layers *.Cu *.Mask) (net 10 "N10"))
  (pad "1" thru_hole rect (at 0 0) (size 1.6 1.6) (drill 0.8) (layers *.Cu *.Mask) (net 2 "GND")))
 (gr_arc (start 161.925 99.695) (end 161.925 100.965) (angle -90) (layer "Edge.Cuts") (width 0.05))
 (gr_arc (start 125.73 99.695) (end 124.46 99.695) (angle -90) (layer "Edge.Cuts") (width 0.05))
 (gr_arc (start 125.73 83.82) (end 125.73 82.55) (angle -90) (layer "Edge.Cuts") (width 0.05))
 (gr_arc (start 161.925 83.82) (end 163.195 83.82) (angle -90) (layer "Edge.Cuts") (width 0.05))
 (gr_line (start 163.195 99.695) (end 163.195 83.82) (layer "Edge.Cuts") (width 0.05))
 (gr_line (start 125.73 100.965) (end 161.925 100.965) (layer "Edge.Cuts") (width 0.05))
 (gr_line (start 125.73 82.55) (end 161.925 82.55) (layer "Edge.Cuts") (width 0.05))
 (gr_line (start 124.46 83.82) (end 124.46 99.695) (layer "Edge.Cuts") (width 0.05))
 (segment (start 131.9703 86.1056) (end 131.9703 85.305) (width 0.25) (layer "B.Cu") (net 10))
 (segment (start 139.2097 93.345) (end 131.9703 86.1056) (width 0.25) (layer "B.Cu") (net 10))
 (segment (start 140.335 93.345) (end 139.2097 93.345) (width 0.25) (layer "B.Cu") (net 10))
 (segment (start 130.795 85.305) (end 131.9703 85.305) (width 0.25) (layer "B.Cu") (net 10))
 (segment (start 141.605 95.7403) (end 140.335 94.4703) (width 0.25) (layer "B.Cu") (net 10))
 (segment (start 141.605 97.79) (end 141.605 95.7403) (width 0.25) (layer "B.Cu") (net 10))
 (segment (start 140.335 93.345) (end 140.335 94.4703) (width 0.25) (layer "B.Cu") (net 10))
 (segment (start 144.145 95.7403) (end 142.875 94.4703) (width 0.25) (layer "B.Cu") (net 8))
 (segment (start 144.145 97.79) (end 144.145 95.7403) (width 0.25) (layer "B.Cu") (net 8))
 (segment (start 142.875 93.345) (end 142.875 94.4703) (width 0.25) (layer "B.Cu") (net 8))
 (segment (start 136.953 87.845) (end 130.795 87.845) (width 0.25) (layer "F.Cu") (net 8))
 (segment (start 141.7497 92.6417) (end 136.953 87.845) (width 0.25) (layer "F.Cu") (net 8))
 (segment (start 141.7497 93.345) (end 141.7497 92.6417) (width 0.25) (layer "F.Cu") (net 8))
 (segment (start 142.875 93.345) (end 141.7497 93.345) (width 0.25) (layer "F.Cu") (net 8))
 (segment (start 146.685 95.7403) (end 145.415 94.4703) (width 0.25) (layer "B.Cu") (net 6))
 (segment (start 146.685 97.79) (end 146.685 95.7403) (width 0.25) (layer "B.Cu") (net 6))
 (segment (start 145.415 93.345) (end 145.415 94.4703) (width 0.25) (layer "B.Cu") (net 6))
 (segment (start 145.415 93.345) (end 144.2897 93.345) (width 0.25) (layer "F.Cu") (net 6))
 (segment (start 130.795 90.385) (end 131.9703 90.385) (width 0.25) (layer "F.Cu") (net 6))
 (segment (start 133.2442 90.385) (end 131.9703 90.385) (width 0.25) (layer "F.Cu") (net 6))
 (segment (start 137.3779 94.5187) (end 133.2442 90.385) (width 0.25) (layer "F.Cu") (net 6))
 (segment (start 143.3973 94.5187) (end 137.3779 94.5187) (width 0.25) (layer "F.Cu") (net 6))
 (segment (start 144.2897 93.6263) (end 143.3973 94.5187) (width 0.25) (layer "F.Cu") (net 6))
 (segment (start 144.2897 93.345) (end 144.2897 93.6263) (width 0.25) (layer "F.Cu") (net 6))
 (segment (start 147.955 93.345) (end 147.955 94.4703) (width 0.25) (layer "B.Cu") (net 4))
 (segment (start 149.225 95.7403) (end 149.225 97.79) (width 0.25) (layer "B.Cu") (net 4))
 (segment (start 147.955 94.4703) (end 149.225 95.7403) (width 0.25) (layer "B.Cu") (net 4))
 (segment (start 138.0643 99.019) (end 131.9703 92.925) (width 0.25) (layer "B.Cu") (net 4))
 (segment (start 147.152 99.019) (end 138.0643 99.019) (width 0.25) (layer "B.Cu") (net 4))
 (segment (start 148.0997 98.0713) (end 147.152 99.019) (width 0.25) (layer "B.Cu") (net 4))
 (segment (start 148.0997 97.79) (end 148.0997 98.0713) (width 0.25) (layer "B.Cu") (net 4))
 (segment (start 149.225 97.79) (end 148.0997 97.79) (width 0.25) (layer "B.Cu") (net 4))
 (segment (start 130.795 92.925) (end 131.9703 92.925) (width 0.25) (layer "B.Cu") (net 4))
 (segment (start 129.4303 84.4969) (end 129.4303 85.305) (width 0.25) (layer "B.Cu") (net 9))
 (segment (start 129.7975 84.1297) (end 129.4303 84.4969) (width 0.25) (layer "B.Cu") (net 9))
 (segment (start 134.0556 84.1297) (end 129.7975 84.1297) (width 0.25) (layer "B.Cu") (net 9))
 (segment (start 142.1456 92.2197) (end 134.0556 84.1297) (width 0.25) (layer "B.Cu") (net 9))
 (segment (start 148.5258 92.2197) (end 142.1456 92.2197) (width 0.25) (layer "B.Cu") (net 9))
 (segment (start 149.3697 93.0636) (end 148.5258 92.2197) (width 0.25) (layer "B.Cu") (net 9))
 (segment (start 149.3697 93.345) (end 149.3697 93.0636) (width 0.25) (layer "B.Cu") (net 9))
 (segment (start 150.495 93.345) (end 149.3697 93.345) (width 0.25) (layer "B.Cu") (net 9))
 (segment (start 128.255 85.305) (end 129.4303 85.305) (width 0.25) (layer "B.Cu") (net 9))
 (segment (start 151.765 95.7403) (end 150.495 94.4703) (width 0.25) (layer "B.Cu") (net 9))
 (segment (start 151.765 97.79) (end 151.765 95.7403) (width 0.25) (layer "B.Cu") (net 9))
 (segment (start 150.495 93.345) (end 150.495 94.4703) (width 0.25) (layer "B.Cu") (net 9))
 (segment (start 154.305 95.7403) (end 153.035 94.4703) (width 0.25) (layer "B.Cu") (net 7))
 (segment (start 154.305 97.79) (end 154.305 95.7403) (width 0.25) (layer "B.Cu") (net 7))
 (segment (start 153.035 93.345) (end 153.035 94.4703) (width 0.25) (layer "B.Cu") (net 7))
 (segment (start 129.4303 87.4776) (end 129.4303 87.845) (width 0.25) (layer "F.Cu") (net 7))
 (segment (start 130.2382 86.6697) (end 129.4303 87.4776) (width 0.25) (layer "F.Cu") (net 7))
 (segment (start 131.5199 86.6697) (end 130.2382 86.6697) (width 0.25) (layer "F.Cu") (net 7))
 (segment (start 131.8899 87.0397) (end 131.5199 86.6697) (width 0.25) (layer "F.Cu") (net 7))
 (segment (start 145.8857 87.0397) (end 131.8899 87.0397) (width 0.25) (layer "F.Cu") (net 7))
 (segment (start 151.9097 93.0637) (end 145.8857 87.0397) (width 0.25) (layer "F.Cu") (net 7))
 (segment (start 151.9097 93.345) (end 151.9097 93.0637) (width 0.25) (layer "F.Cu") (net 7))
 (segment (start 153.035 93.345) (end 151.9097 93.345) (width 0.25) (layer "F.Cu") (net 7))
 (segment (start 128.255 87.845) (end 129.4303 87.845) (width 0.25) (layer "F.Cu") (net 7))
 (segment (start 156.845 95.7403) (end 155.575 94.4703) (width 0.25) (layer "B.Cu") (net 5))
 (segment (start 156.845 97.79) (end 156.845 95.7403) (width 0.25) (layer "B.Cu") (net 5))
 (segment (start 155.575 93.345) (end 155.575 94.4703) (width 0.25) (layer "B.Cu") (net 5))
 (segment (start 155.575 93.345) (end 154.4497 93.345) (width 0.25) (layer "F.Cu") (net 5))
 (segment (start 128.255 90.385) (end 129.4303 90.385) (width 0.25) (layer "F.Cu") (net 5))
 (segment (start 129.4303 90.7524) (end 129.4303 90.385) (width 0.25) (layer "F.Cu") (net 5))
 (segment (start 130.2382 91.5603) (end 129.4303 90.7524) (width 0.25) (layer "F.Cu") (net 5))
 (segment (start 133.7826 91.5603) (end 130.2382 91.5603) (width 0.25) (layer "F.Cu") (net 5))
 (segment (start 137.1914 94.9691) (end 133.7826 91.5603) (width 0.25) (layer "F.Cu") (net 5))
 (segment (start 153.1069 94.9691) (end 137.1914 94.9691) (width 0.25) (layer "F.Cu") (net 5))
 (segment (start 154.4497 93.6263) (end 153.1069 94.9691) (width 0.25) (layer "F.Cu") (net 5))
 (segment (start 154.4497 93.345) (end 154.4497 93.6263) (width 0.25) (layer "F.Cu") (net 5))
 (segment (start 159.385 95.7403) (end 158.115 94.4703) (width 0.25) (layer "B.Cu") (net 3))
 (segment (start 159.385 97.79) (end 159.385 95.7403) (width 0.25) (layer "B.Cu") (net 3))
 (segment (start 158.115 93.345) (end 158.115 94.4703) (width 0.25) (layer "B.Cu") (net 3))
 (segment (start 129.4303 93.2924) (end 129.4303 92.925) (width 0.25) (layer "F.Cu") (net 3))
 (segment (start 130.2382 94.1003) (end 129.4303 93.2924) (width 0.25) (layer "F.Cu") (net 3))
 (segment (start 133.3667 94.1003) (end 130.2382 94.1003) (width 0.25) (layer "F.Cu") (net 3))
 (segment (start 134.6859 95.4195) (end 133.3667 94.1003) (width 0.25) (layer "F.Cu") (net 3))
 (segment (start 155.1965 95.4195) (end 134.6859 95.4195) (width 0.25) (layer "F.Cu") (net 3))
 (segment (start 156.9897 93.6263) (end 155.1965 95.4195) (width 0.25) (layer "F.Cu") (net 3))
 (segment (start 156.9897 93.345) (end 156.9897 93.6263) (width 0.25) (layer "F.Cu") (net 3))
 (segment (start 158.115 93.345) (end 156.9897 93.345) (width 0.25) (layer "F.Cu") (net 3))
 (segment (start 128.255 92.925) (end 129.4303 92.925) (width 0.25) (layer "F.Cu") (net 3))
 (segment (start 139.065 97.79) (end 137.7147 97.79) (width 0.5) (layer "F.Cu") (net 2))
 (segment (start 134.5203 97.79) (end 137.7147 97.79) (width 0.5) (layer "F.Cu") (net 2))
 (segment (start 132.1953 95.465) (end 134.5203 97.79) (width 0.5) (layer "F.Cu") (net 2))
 (segment (start 131.0044 95.465) (end 132.1953 95.465) (width 0.5) (layer "F.Cu") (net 2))
 (segment (start 131.0044 95.465) (end 130.795 95.465) (width 0.5) (layer "F.Cu") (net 2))
 (segment (start 130.795 95.465) (end 128.255 95.465) (width 0.5) (layer "F.Cu") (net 2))
 (segment (start 158.115 85.725) (end 155.575 85.725) (width 0.5) (layer "F.Cu") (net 1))
 (segment (start 155.575 85.725) (end 153.035 85.725) (width 0.5) (layer "F.Cu") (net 1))
 (segment (start 153.035 85.725) (end 150.495 85.725) (width 0.5) (layer "B.Cu") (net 1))
 (segment (start 150.495 85.725) (end 147.955 85.725) (width 0.5) (layer "B.Cu") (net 1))
 (segment (start 147.955 85.725) (end 145.415 85.725) (width 0.5) (layer "F.Cu") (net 1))
 (segment (start 145.415 85.725) (end 142.875 85.725) (width 0.5) (layer "F.Cu") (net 1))
 (segment (start 142.875 85.725) (end 140.335 85.725) (width 0.5) (layer "F.Cu") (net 1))
 (segment (start 126.8534 96.6034) (end 128.255 98.005) (width 0.5) (layer "B.Cu") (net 1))
 (segment (start 126.8534 84.7258) (end 126.8534 96.6034) (width 0.5) (layer "B.Cu") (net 1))
 (segment (start 128.1775 83.4017) (end 126.8534 84.7258) (width 0.5) (layer "B.Cu") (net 1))
 (segment (start 136.6614 83.4017) (end 128.1775 83.4017) (width 0.5) (layer "B.Cu") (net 1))
 (segment (start 138.9847 85.725) (end 136.6614 83.4017) (width 0.5) (layer "B.Cu") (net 1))
 (segment (start 140.335 85.725) (end 138.9847 85.725) (width 0.5) (layer "B.Cu") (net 1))
 (segment (start 130.795 98.005) (end 128.255 98.005) (width 0.5) (layer "F.Cu") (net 1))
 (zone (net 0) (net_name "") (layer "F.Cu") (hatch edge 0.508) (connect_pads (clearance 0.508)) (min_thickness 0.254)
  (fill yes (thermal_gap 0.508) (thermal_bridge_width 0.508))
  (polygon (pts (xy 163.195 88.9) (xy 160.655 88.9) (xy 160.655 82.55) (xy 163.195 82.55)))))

